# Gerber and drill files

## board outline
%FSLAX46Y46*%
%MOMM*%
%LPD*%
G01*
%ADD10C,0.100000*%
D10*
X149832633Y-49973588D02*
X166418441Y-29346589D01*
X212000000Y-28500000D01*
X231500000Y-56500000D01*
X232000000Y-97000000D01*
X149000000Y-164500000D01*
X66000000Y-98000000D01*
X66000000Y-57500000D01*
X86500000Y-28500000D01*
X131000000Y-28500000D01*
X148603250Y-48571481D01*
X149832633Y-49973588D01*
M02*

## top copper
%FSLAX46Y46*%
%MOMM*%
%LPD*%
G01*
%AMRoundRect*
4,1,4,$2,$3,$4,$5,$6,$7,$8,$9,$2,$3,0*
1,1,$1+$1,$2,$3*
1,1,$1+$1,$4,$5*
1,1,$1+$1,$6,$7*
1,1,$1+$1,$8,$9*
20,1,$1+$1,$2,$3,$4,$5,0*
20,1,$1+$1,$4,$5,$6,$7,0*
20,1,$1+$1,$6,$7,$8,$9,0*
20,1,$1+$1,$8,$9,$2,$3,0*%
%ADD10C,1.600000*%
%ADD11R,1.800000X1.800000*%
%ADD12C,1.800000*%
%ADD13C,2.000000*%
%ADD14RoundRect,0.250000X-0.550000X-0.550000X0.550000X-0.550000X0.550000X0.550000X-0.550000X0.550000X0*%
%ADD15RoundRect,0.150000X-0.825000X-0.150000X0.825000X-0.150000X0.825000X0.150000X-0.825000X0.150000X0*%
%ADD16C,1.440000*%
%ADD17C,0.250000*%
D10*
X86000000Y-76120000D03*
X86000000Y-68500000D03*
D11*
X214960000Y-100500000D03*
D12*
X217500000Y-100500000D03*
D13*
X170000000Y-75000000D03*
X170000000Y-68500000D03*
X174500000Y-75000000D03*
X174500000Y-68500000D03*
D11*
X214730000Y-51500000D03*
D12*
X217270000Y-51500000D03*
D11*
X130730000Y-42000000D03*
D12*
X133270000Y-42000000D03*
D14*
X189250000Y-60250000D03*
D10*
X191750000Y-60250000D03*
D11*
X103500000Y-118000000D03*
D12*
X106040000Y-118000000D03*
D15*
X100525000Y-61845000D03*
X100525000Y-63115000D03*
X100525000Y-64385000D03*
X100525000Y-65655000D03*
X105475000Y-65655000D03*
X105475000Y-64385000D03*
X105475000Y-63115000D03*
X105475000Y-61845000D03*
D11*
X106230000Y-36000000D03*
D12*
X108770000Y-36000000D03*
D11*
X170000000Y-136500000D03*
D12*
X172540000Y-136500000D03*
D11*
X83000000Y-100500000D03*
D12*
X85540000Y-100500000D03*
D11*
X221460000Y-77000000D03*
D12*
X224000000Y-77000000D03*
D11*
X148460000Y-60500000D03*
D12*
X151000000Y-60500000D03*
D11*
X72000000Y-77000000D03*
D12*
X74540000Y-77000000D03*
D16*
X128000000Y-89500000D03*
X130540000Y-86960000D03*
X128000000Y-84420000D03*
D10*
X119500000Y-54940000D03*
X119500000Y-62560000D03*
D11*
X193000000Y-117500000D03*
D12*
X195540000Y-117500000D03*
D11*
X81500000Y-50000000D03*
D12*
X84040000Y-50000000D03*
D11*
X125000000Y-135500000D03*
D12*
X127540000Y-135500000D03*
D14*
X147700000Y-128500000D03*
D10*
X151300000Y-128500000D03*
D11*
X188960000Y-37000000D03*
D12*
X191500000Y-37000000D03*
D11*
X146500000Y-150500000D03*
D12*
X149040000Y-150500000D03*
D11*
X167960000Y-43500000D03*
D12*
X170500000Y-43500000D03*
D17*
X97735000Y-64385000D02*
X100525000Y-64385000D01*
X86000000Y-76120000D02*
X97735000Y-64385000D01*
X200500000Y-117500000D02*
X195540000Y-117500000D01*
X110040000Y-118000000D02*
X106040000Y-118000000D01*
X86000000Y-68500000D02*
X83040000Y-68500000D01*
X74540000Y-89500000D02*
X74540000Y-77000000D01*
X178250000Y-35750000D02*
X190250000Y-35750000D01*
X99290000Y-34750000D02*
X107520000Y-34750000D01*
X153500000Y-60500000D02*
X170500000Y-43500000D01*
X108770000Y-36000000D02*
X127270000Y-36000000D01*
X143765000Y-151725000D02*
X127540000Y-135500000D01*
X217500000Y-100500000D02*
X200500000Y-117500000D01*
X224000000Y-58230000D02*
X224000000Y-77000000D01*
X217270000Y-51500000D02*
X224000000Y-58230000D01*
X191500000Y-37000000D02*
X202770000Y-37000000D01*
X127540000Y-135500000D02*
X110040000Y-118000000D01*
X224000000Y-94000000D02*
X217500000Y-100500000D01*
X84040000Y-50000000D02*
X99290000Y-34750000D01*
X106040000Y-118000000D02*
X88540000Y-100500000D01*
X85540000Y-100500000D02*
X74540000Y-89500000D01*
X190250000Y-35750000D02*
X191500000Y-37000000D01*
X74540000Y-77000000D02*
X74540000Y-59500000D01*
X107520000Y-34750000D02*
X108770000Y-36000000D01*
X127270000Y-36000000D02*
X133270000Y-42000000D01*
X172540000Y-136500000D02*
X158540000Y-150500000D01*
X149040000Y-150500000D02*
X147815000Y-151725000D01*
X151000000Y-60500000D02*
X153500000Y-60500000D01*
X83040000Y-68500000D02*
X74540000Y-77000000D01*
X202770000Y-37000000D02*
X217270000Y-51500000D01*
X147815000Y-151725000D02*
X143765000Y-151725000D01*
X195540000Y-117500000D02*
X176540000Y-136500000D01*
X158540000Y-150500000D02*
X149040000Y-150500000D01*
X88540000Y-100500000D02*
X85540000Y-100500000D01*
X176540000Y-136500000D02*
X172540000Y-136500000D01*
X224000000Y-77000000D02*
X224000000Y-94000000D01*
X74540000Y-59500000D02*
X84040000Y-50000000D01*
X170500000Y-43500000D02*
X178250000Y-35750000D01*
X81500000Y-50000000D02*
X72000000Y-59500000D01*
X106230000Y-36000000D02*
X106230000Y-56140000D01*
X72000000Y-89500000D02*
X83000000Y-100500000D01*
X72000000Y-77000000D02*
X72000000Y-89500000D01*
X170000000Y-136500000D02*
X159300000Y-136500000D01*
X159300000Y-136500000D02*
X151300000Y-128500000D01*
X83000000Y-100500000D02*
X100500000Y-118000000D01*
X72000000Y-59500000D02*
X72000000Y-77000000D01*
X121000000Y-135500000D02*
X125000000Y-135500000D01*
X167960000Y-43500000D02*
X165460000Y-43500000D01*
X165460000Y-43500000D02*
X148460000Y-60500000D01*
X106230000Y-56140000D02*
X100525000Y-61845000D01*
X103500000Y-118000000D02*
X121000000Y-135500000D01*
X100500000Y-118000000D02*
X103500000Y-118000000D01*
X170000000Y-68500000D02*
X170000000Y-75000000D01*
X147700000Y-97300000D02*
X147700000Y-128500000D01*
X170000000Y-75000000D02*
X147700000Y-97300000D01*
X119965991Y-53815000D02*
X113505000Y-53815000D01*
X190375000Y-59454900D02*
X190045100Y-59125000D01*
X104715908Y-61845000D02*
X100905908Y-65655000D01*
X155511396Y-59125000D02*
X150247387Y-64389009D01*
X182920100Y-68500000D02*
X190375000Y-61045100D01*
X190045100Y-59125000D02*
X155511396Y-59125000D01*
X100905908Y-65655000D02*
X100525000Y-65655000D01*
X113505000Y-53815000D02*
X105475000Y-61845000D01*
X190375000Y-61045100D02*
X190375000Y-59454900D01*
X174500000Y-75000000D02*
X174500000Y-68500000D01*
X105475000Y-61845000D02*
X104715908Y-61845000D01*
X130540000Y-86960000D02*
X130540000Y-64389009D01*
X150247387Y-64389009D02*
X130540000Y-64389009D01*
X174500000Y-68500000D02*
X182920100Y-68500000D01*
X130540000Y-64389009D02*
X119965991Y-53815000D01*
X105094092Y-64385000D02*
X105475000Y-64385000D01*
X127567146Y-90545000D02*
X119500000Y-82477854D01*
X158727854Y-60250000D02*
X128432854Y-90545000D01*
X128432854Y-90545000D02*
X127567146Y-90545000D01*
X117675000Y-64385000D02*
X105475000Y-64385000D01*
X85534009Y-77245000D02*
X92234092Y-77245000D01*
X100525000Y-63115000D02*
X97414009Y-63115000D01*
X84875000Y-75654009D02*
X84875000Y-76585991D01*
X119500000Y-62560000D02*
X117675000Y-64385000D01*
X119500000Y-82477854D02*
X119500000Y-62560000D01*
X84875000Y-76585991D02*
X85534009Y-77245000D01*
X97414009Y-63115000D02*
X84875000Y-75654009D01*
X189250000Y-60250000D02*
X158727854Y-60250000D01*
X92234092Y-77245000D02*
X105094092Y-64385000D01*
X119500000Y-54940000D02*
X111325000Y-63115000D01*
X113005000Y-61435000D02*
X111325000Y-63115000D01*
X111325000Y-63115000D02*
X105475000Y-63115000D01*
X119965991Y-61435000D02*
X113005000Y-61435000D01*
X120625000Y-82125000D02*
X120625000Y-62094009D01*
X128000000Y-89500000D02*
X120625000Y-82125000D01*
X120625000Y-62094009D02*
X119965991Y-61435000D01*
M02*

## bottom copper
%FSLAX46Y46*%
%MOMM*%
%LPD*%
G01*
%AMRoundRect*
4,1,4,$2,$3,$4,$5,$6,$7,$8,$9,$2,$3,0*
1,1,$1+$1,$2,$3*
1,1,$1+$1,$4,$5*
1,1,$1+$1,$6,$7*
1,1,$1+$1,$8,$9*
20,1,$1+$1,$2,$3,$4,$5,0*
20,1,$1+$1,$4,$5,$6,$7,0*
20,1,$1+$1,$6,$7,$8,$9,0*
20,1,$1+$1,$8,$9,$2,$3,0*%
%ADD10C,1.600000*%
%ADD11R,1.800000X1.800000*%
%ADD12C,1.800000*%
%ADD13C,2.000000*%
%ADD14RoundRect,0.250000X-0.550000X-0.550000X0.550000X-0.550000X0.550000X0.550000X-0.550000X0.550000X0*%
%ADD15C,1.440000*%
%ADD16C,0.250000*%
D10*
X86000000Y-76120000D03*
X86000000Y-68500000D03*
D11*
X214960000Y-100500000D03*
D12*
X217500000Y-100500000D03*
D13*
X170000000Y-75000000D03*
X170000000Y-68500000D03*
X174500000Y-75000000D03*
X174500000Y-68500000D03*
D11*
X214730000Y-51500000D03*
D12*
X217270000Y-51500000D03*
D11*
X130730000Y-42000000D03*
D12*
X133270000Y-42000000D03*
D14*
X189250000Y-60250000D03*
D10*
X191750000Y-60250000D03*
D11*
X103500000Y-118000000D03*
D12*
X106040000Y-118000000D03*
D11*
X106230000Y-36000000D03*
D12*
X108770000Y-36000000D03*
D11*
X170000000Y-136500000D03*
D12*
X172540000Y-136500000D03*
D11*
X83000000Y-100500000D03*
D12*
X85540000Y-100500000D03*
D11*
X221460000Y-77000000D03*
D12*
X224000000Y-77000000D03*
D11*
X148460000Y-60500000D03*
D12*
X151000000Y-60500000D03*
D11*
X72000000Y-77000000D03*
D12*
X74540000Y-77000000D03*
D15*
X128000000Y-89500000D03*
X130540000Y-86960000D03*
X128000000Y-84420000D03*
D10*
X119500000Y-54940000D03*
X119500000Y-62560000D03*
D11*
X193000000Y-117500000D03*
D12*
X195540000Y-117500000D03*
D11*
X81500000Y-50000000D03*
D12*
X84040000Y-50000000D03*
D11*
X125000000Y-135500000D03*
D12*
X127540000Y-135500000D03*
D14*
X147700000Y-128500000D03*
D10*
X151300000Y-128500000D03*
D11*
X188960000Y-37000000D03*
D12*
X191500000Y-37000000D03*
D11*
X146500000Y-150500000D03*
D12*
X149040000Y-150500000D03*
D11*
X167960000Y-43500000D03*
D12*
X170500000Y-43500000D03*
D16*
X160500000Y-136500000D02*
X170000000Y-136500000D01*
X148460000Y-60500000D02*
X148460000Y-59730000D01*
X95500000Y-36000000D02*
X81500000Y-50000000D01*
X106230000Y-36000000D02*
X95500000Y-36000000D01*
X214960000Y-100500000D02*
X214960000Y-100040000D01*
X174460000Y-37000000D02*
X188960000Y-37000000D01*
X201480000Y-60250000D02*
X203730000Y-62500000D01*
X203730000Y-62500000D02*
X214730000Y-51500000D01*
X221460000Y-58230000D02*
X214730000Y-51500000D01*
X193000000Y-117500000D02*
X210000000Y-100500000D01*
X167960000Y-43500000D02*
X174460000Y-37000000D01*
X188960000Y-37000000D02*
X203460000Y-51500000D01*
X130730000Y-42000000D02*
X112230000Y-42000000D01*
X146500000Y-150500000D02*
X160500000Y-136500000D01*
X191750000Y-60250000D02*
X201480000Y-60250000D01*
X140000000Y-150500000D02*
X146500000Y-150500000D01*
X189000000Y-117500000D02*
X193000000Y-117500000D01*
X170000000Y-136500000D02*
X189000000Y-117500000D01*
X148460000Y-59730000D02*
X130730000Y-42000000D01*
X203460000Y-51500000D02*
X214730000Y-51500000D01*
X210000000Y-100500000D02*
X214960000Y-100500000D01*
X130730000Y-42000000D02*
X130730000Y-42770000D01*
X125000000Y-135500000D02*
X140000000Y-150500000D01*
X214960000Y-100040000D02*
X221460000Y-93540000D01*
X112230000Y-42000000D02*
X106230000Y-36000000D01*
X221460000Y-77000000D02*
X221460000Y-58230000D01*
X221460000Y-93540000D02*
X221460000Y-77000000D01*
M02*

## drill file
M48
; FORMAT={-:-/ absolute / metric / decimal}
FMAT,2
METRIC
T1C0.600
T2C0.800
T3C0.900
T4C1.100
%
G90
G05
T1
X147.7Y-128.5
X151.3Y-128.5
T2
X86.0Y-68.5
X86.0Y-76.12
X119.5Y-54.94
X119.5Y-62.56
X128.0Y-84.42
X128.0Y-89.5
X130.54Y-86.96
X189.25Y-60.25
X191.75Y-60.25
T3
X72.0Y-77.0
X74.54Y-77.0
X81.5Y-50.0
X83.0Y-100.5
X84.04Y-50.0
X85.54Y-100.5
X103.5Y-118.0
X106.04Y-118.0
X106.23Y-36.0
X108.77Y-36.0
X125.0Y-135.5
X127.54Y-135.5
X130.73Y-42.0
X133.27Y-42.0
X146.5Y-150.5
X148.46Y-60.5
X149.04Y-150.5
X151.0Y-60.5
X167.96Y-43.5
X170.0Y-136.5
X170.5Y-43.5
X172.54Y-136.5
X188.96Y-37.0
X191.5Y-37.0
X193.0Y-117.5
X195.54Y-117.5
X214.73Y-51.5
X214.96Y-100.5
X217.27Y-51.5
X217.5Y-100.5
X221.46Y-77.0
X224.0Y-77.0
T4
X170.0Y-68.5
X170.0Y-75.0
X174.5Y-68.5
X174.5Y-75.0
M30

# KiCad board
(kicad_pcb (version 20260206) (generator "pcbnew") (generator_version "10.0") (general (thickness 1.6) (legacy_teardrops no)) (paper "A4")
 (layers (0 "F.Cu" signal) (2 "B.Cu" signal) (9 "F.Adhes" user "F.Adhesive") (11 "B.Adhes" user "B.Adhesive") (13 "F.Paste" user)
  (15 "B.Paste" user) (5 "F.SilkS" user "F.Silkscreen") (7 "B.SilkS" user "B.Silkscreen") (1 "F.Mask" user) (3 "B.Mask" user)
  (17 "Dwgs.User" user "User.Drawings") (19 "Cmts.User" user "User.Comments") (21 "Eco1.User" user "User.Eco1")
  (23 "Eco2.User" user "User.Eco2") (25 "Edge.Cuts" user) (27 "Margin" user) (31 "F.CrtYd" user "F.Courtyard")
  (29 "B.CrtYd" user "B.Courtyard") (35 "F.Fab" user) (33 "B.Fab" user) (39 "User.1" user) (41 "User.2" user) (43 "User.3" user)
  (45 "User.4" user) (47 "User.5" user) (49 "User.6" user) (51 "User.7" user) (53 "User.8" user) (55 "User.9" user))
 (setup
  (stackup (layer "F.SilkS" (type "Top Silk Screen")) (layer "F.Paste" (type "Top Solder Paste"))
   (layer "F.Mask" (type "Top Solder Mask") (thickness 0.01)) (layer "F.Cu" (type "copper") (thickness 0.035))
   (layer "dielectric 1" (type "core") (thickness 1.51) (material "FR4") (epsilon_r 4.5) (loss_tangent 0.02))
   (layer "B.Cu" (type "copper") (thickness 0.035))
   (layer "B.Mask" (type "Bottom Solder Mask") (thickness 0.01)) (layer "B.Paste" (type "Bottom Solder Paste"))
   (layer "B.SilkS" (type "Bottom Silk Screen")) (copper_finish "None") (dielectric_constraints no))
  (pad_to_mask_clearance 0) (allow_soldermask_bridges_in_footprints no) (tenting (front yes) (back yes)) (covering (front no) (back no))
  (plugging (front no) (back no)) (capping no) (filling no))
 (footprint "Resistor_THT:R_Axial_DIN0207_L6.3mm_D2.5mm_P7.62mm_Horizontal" (layer "F.Cu") (at 86 76.12 90)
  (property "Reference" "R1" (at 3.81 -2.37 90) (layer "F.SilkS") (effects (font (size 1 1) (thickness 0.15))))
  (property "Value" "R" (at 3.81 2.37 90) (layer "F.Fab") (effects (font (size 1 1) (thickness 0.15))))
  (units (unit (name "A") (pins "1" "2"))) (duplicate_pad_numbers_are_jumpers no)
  (pad "1" thru_hole circle (at 0 0 90) (size 1.6 1.6) (drill 0.8) (layers "*.Cu" "*.Mask") (remove_unused_layers no) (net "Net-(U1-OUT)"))
  (pad "2" thru_hole circle (at 7.62 0 90) (size 1.6 1.6) (drill 0.8) (layers "*.Cu" "*.Mask") (remove_unused_layers no) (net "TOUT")))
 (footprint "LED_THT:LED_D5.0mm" (layer "F.Cu") (at 214.96 100.5)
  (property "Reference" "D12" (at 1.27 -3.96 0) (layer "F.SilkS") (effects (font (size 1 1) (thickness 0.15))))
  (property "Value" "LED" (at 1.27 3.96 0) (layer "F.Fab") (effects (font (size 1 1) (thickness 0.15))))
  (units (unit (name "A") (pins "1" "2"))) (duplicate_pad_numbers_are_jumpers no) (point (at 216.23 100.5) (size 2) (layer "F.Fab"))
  (pad "1" thru_hole rect (at 0 0) (size 1.8 1.8) (drill 0.9) (layers "*.Cu" "*.Mask") (remove_unused_layers no) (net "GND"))
  (pad "2" thru_hole circle (at 2.54 0) (size 1.8 1.8) (drill 0.9) (layers "*.Cu" "*.Mask") (remove_unused_layers no) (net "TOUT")))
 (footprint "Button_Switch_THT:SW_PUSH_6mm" (layer "F.Cu") (at 170 75 90)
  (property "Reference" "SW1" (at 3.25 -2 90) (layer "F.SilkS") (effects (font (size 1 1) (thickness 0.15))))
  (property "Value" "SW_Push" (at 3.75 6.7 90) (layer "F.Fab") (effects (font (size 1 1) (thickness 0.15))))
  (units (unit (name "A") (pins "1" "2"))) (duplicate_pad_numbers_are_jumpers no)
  (pad "1" thru_hole circle (at 0 0 180) (size 2 2) (drill 1.1) (layers "*.Cu" "*.Mask") (remove_unused_layers no) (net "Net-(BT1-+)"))
  (pad "1" thru_hole circle (at 6.5 0 180) (size 2 2) (drill 1.1) (layers "*.Cu" "*.Mask") (remove_unused_layers no) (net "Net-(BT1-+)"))
  (pad "2" thru_hole circle (at 0 4.5 180) (size 2 2) (drill 1.1) (layers "*.Cu" "*.Mask") (remove_unused_layers no) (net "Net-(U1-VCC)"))
  (pad "2" thru_hole circle (at 6.5 4.5 180) (size 2 2) (drill 1.1) (layers "*.Cu" "*.Mask") (remove_unused_layers no) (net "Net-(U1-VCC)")))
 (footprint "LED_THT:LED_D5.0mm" (layer "F.Cu") (at 214.73 51.5)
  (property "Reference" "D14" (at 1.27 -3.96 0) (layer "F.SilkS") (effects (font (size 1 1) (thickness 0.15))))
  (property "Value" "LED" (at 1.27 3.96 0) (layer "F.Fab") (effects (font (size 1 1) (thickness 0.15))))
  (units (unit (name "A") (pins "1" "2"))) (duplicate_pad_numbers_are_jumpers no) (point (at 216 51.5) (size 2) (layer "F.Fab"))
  (pad "1" thru_hole rect (at 0 0) (size 1.8 1.8) (drill 0.9) (layers "*.Cu" "*.Mask") (remove_unused_layers no) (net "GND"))
  (pad "2" thru_hole circle (at 2.54 0) (size 1.8 1.8) (drill 0.9) (layers "*.Cu" "*.Mask") (remove_unused_layers no) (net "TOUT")))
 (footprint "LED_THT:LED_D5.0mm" (layer "F.Cu") (at 130.73 42)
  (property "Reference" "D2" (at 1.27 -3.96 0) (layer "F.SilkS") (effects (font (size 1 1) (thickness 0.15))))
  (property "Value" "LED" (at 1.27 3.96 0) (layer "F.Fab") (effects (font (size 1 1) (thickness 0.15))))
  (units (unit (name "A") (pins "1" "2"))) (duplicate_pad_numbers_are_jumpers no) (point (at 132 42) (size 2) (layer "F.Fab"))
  (pad "1" thru_hole rect (at 0 0) (size 1.8 1.8) (drill 0.9) (layers "*.Cu" "*.Mask") (remove_unused_layers no) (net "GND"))
  (pad "2" thru_hole circle (at 2.54 0) (size 1.8 1.8) (drill 0.9) (layers "*.Cu" "*.Mask") (remove_unused_layers no) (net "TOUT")))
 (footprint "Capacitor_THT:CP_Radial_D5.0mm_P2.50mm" (layer "F.Cu") (at 189.25 60.25)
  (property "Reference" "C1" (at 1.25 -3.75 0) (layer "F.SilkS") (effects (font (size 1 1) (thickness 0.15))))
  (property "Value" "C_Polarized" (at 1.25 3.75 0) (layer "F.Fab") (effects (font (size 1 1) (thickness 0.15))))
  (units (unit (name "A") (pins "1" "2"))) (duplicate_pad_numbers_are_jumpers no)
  (pad "1" thru_hole roundrect (at 0 0) (size 1.6 1.6) (drill 0.8) (layers "*.Cu" "*.Mask") (remove_unused_layers no)
   (roundrect_rratio 0.15625) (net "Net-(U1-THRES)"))
  (pad "2" thru_hole circle (at 2.5 0) (size 1.6 1.6) (drill 0.8) (layers "*.Cu" "*.Mask") (remove_unused_layers no) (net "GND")))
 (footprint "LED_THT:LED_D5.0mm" (layer "F.Cu") (at 103.5 118)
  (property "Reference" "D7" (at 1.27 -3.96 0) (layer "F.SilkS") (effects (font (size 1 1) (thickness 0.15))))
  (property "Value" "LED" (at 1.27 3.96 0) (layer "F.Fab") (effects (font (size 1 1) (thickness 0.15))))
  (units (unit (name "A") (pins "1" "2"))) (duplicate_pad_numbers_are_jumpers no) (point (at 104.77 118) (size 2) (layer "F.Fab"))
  (pad "1" thru_hole rect (at 0 0) (size 1.8 1.8) (drill 0.9) (layers "*.Cu" "*.Mask") (remove_unused_layers no) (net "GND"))
  (pad "2" thru_hole circle (at 2.54 0) (size 1.8 1.8) (drill 0.9) (layers "*.Cu" "*.Mask") (remove_unused_layers no) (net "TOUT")))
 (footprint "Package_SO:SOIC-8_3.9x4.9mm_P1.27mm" (layer "F.Cu") (at 103 63.75)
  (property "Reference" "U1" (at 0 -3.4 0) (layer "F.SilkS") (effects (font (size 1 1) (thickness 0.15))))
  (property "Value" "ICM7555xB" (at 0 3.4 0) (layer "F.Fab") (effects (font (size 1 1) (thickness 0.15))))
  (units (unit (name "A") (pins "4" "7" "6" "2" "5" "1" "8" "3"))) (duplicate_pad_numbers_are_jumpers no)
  (pad "1" smd roundrect (at -2.475 -1.905) (size 1.95 0.6) (layers "F.Cu" "F.Mask" "F.Paste") (roundrect_rratio 0.25) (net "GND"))
  (pad "2" smd roundrect (at -2.475 -0.635) (size 1.95 0.6) (layers "F.Cu" "F.Mask" "F.Paste") (roundrect_rratio 0.25)
   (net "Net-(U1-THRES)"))
  (pad "3" smd roundrect (at -2.475 0.635) (size 1.95 0.6) (layers "F.Cu" "F.Mask" "F.Paste") (roundrect_rratio 0.25) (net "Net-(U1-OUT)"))
  (pad "4" smd roundrect (at -2.475 1.905) (size 1.95 0.6) (layers "F.Cu" "F.Mask" "F.Paste") (roundrect_rratio 0.25) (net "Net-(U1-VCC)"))
  (pad "5" smd roundrect (at 2.475 1.905) (size 1.95 0.6) (layers "F.Cu" "F.Mask" "F.Paste") (roundrect_rratio 0.25)
   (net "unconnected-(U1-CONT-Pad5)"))
  (pad "6" smd roundrect (at 2.475 0.635) (size 1.95 0.6) (layers "F.Cu" "F.Mask" "F.Paste") (roundrect_rratio 0.25) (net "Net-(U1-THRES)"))
  (pad "7" smd roundrect (at 2.475 -0.635) (size 1.95 0.6) (layers "F.Cu" "F.Mask" "F.Paste") (roundrect_rratio 0.25) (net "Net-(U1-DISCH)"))
  (pad "8" smd roundrect (at 2.475 -1.905) (size 1.95 0.6) (layers "F.Cu" "F.Mask" "F.Paste") (roundrect_rratio 0.25) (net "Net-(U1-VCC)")))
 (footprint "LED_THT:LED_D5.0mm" (layer "F.Cu") (at 106.23 36)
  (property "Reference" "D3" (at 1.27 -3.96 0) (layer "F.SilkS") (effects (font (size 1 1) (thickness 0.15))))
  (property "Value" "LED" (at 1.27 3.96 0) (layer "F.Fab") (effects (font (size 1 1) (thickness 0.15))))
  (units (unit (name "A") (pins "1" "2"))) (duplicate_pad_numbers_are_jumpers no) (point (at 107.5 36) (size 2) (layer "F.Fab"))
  (pad "1" thru_hole rect (at 0 0) (size 1.8 1.8) (drill 0.9) (layers "*.Cu" "*.Mask") (remove_unused_layers no) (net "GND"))
  (pad "2" thru_hole circle (at 2.54 0) (size 1.8 1.8) (drill 0.9) (layers "*.Cu" "*.Mask") (remove_unused_layers no) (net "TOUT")))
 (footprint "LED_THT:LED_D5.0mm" (layer "F.Cu") (at 170 136.5)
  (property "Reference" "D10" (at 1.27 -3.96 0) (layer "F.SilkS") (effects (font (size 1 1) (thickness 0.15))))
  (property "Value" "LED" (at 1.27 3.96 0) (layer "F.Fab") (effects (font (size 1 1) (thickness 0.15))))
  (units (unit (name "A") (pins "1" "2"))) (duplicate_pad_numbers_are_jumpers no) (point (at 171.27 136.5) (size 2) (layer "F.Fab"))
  (pad "1" thru_hole rect (at 0 0) (size 1.8 1.8) (drill 0.9) (layers "*.Cu" "*.Mask") (remove_unused_layers no) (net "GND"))
  (pad "2" thru_hole circle (at 2.54 0) (size 1.8 1.8) (drill 0.9) (layers "*.Cu" "*.Mask") (remove_unused_layers no) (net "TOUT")))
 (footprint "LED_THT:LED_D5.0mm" (layer "F.Cu") (at 83 100.5)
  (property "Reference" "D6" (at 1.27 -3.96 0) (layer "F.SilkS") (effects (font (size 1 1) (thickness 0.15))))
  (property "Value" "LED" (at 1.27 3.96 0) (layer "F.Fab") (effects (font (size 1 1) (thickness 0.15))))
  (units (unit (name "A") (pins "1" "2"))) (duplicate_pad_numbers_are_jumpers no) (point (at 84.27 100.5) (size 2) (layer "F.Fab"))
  (pad "1" thru_hole rect (at 0 0) (size 1.8 1.8) (drill 0.9) (layers "*.Cu" "*.Mask") (remove_unused_layers no) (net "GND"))
  (pad "2" thru_hole circle (at 2.54 0) (size 1.8 1.8) (drill 0.9) (layers "*.Cu" "*.Mask") (remove_unused_layers no) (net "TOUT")))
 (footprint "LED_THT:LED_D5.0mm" (layer "F.Cu") (at 221.46 77)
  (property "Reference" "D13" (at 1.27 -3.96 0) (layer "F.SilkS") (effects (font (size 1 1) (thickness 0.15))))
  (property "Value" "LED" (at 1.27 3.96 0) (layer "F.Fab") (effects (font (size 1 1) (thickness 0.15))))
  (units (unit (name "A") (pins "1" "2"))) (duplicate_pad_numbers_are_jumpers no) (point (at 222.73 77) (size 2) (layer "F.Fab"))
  (pad "1" thru_hole rect (at 0 0) (size 1.8 1.8) (drill 0.9) (layers "*.Cu" "*.Mask") (remove_unused_layers no) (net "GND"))
  (pad "2" thru_hole circle (at 2.54 0) (size 1.8 1.8) (drill 0.9) (layers "*.Cu" "*.Mask") (remove_unused_layers no) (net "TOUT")))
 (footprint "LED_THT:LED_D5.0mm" (layer "F.Cu") (at 148.46 60.5)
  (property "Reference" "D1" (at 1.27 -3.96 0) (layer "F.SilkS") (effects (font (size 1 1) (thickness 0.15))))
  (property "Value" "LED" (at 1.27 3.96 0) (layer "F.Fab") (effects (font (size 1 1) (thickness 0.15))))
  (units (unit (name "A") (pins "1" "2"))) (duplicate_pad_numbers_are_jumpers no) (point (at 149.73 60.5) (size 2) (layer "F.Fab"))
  (pad "1" thru_hole rect (at 0 0) (size 1.8 1.8) (drill 0.9) (layers "*.Cu" "*.Mask") (remove_unused_layers no) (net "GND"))
  (pad "2" thru_hole circle (at 2.54 0) (size 1.8 1.8) (drill 0.9) (layers "*.Cu" "*.Mask") (remove_unused_layers no) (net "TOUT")))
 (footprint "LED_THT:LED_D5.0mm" (layer "F.Cu") (at 72 77)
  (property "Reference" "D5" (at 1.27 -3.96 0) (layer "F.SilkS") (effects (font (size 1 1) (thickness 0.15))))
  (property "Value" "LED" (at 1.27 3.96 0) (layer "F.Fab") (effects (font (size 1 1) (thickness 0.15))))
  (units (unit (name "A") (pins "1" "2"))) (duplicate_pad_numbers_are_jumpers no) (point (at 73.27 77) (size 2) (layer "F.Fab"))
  (pad "1" thru_hole rect (at 0 0) (size 1.8 1.8) (drill 0.9) (layers "*.Cu" "*.Mask") (remove_unused_layers no) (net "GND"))
  (pad "2" thru_hole circle (at 2.54 0) (size 1.8 1.8) (drill 0.9) (layers "*.Cu" "*.Mask") (remove_unused_layers no) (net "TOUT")))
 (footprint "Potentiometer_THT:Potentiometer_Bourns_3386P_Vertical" (layer "F.Cu") (at 128 89.5)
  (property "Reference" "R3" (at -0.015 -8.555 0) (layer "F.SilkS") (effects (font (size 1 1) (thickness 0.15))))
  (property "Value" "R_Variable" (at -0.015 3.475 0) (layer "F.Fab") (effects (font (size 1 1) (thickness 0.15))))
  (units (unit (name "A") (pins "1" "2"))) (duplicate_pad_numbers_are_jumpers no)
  (pad "1" thru_hole circle (at 0 0) (size 1.44 1.44) (drill 0.8) (layers "*.Cu" "*.Mask") (remove_unused_layers no) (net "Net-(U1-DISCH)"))
  (pad "2" thru_hole circle (at 2.54 -2.54) (size 1.44 1.44) (drill 0.8) (layers "*.Cu" "*.Mask") (remove_unused_layers no)
   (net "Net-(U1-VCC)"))
  (pad "3" thru_hole circle (at 0 -5.08) (size 1.44 1.44) (drill 0.8) (layers "*.Cu" "*.Mask") (remove_unused_layers no)))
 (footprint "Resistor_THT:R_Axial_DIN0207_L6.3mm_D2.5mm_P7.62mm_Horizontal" (layer "F.Cu") (at 119.5 54.94 -90)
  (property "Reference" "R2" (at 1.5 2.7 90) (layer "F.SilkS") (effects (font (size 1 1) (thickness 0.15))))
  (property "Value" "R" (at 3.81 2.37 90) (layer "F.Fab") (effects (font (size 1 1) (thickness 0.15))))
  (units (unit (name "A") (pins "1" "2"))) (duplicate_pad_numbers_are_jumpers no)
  (pad "1" thru_hole circle (at 0 0 270) (size 1.6 1.6) (drill 0.8) (layers "*.Cu" "*.Mask") (remove_unused_layers no)
   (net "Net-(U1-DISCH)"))
  (pad "2" thru_hole circle (at 7.62 0 270) (size 1.6 1.6) (drill 0.8) (layers "*.Cu" "*.Mask") (remove_unused_layers no)
   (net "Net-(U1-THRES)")))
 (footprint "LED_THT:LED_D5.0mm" (layer "F.Cu") (at 193 117.5)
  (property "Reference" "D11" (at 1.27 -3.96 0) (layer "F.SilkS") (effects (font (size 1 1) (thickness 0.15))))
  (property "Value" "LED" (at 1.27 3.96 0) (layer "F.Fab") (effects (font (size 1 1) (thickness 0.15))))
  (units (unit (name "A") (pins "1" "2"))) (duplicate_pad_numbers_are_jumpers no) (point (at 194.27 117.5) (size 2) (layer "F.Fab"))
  (pad "1" thru_hole rect (at 0 0) (size 1.8 1.8) (drill 0.9) (layers "*.Cu" "*.Mask") (remove_unused_layers no) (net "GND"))
  (pad "2" thru_hole circle (at 2.54 0) (size 1.8 1.8) (drill 0.9) (layers "*.Cu" "*.Mask") (remove_unused_layers no) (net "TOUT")))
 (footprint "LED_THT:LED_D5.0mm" (layer "F.Cu") (at 81.5 50)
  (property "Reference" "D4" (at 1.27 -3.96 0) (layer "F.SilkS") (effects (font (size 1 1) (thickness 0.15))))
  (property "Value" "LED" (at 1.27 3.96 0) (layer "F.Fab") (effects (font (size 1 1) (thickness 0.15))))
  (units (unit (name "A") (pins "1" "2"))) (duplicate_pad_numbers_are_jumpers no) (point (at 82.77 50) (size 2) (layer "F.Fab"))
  (pad "1" thru_hole rect (at 0 0) (size 1.8 1.8) (drill 0.9) (layers "*.Cu" "*.Mask") (remove_unused_layers no) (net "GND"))
  (pad "2" thru_hole circle (at 2.54 0) (size 1.8 1.8) (drill 0.9) (layers "*.Cu" "*.Mask") (remove_unused_layers no) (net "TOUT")))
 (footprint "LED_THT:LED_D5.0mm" (layer "F.Cu") (at 125 135.5)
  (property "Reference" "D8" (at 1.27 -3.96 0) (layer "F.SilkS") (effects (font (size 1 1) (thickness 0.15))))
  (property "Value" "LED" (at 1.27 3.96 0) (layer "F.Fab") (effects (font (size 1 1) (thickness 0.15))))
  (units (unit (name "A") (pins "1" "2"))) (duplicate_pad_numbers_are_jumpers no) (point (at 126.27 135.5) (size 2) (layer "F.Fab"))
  (pad "1" thru_hole rect (at 0 0) (size 1.8 1.8) (drill 0.9) (layers "*.Cu" "*.Mask") (remove_unused_layers no) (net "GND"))
  (pad "2" thru_hole circle (at 2.54 0) (size 1.8 1.8) (drill 0.9) (layers "*.Cu" "*.Mask") (remove_unused_layers no) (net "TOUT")))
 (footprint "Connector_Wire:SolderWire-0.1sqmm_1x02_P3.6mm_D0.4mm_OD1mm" (layer "F.Cu") (at 147.7 128.5)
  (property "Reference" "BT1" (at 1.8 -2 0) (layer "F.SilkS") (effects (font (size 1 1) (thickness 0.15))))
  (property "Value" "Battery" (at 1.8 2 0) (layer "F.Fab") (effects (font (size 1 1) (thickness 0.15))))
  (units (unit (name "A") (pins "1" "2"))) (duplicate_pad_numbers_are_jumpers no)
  (pad "1" thru_hole roundrect (at 0 0) (size 1.6 1.6) (drill 0.6) (layers "*.Cu" "*.Mask") (remove_unused_layers no)
   (roundrect_rratio 0.15625) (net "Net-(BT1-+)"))
  (pad "2" thru_hole circle (at 3.6 0) (size 1.6 1.6) (drill 0.6) (layers "*.Cu" "*.Mask") (remove_unused_layers no) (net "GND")))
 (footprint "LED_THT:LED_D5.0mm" (layer "F.Cu") (at 188.96 37)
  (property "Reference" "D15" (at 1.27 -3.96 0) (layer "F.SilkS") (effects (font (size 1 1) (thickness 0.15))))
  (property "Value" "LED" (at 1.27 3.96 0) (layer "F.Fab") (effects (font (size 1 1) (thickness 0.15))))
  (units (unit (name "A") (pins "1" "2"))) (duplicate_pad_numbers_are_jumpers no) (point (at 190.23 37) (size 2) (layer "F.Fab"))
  (pad "1" thru_hole rect (at 0 0) (size 1.8 1.8) (drill 0.9) (layers "*.Cu" "*.Mask") (remove_unused_layers no) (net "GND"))
  (pad "2" thru_hole circle (at 2.54 0) (size 1.8 1.8) (drill 0.9) (layers "*.Cu" "*.Mask") (remove_unused_layers no) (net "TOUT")))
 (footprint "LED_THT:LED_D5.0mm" (layer "F.Cu") (at 146.5 150.5)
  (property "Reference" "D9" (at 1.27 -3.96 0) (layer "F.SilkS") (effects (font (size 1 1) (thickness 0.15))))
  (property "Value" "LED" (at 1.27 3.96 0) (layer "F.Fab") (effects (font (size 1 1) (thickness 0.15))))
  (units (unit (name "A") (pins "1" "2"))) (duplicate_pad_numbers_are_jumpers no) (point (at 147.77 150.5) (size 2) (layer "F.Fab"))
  (pad "1" thru_hole rect (at 0 0) (size 1.8 1.8) (drill 0.9) (layers "*.Cu" "*.Mask") (remove_unused_layers no) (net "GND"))
  (pad "2" thru_hole circle (at 2.54 0) (size 1.8 1.8) (drill 0.9) (layers "*.Cu" "*.Mask") (remove_unused_layers no) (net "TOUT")))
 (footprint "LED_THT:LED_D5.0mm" (layer "F.Cu") (at 167.96 43.5)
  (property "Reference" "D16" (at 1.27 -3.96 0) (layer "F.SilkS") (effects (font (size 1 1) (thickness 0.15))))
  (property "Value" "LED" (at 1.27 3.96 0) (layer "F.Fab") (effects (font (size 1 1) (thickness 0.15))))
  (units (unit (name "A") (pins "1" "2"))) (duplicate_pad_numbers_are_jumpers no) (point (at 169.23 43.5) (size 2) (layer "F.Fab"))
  (pad "1" thru_hole rect (at 0 0) (size 1.8 1.8) (drill 0.9) (layers "*.Cu" "*.Mask") (remove_unused_layers no) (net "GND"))
  (pad "2" thru_hole circle (at 2.54 0) (size 1.8 1.8) (drill 0.9) (layers "*.Cu" "*.Mask") (remove_unused_layers no) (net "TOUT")))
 (gr_poly
  (pts (xy 149.832633 49.973588) (xy 166.418441 29.346589) (xy 212 28.5) (xy 231.5 56.5) (xy 232 97) (xy 149 164.5) (xy 66 98) (xy 66 57.5)
   (xy 86.5 28.5) (xy 131 28.5) (xy 148.60325 48.571481))
  (stroke (width 0.1) (type solid)) (fill no) (layer "Edge.Cuts"))
 (segment (start 97.735 64.385) (end 100.525 64.385) (width 0.25) (layer "F.Cu") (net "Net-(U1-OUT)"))
 (segment (start 86 76.12) (end 97.735 64.385) (width 0.25) (layer "F.Cu") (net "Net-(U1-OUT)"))
 (segment (start 200.5 117.5) (end 195.54 117.5) (width 0.25) (layer "F.Cu") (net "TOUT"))
 (segment (start 110.04 118) (end 106.04 118) (width 0.25) (layer "F.Cu") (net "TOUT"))
 (segment (start 86 68.5) (end 83.04 68.5) (width 0.25) (layer "F.Cu") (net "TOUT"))
 (segment (start 74.54 89.5) (end 74.54 77) (width 0.25) (layer "F.Cu") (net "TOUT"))
 (segment (start 178.25 35.75) (end 190.25 35.75) (width 0.25) (layer "F.Cu") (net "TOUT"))
 (segment (start 99.29 34.75) (end 107.52 34.75) (width 0.25) (layer "F.Cu") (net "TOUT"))
 (segment (start 153.5 60.5) (end 170.5 43.5) (width 0.25) (layer "F.Cu") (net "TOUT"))
 (segment (start 108.77 36) (end 127.27 36) (width 0.25) (layer "F.Cu") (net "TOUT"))
 (segment (start 143.765 151.725) (end 127.54 135.5) (width 0.25) (layer "F.Cu") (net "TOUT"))
 (segment (start 217.5 100.5) (end 200.5 117.5) (width 0.25) (layer "F.Cu") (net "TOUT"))
 (segment (start 224 58.23) (end 224 77) (width 0.25) (layer "F.Cu") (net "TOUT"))
 (segment (start 217.27 51.5) (end 224 58.23) (width 0.25) (layer "F.Cu") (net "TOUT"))
 (segment (start 191.5 37) (end 202.77 37) (width 0.25) (layer "F.Cu") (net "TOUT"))
 (segment (start 127.54 135.5) (end 110.04 118) (width 0.25) (layer "F.Cu") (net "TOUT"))
 (segment (start 224 94) (end 217.5 100.5) (width 0.25) (layer "F.Cu") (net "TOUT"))
 (segment (start 84.04 50) (end 99.29 34.75) (width 0.25) (layer "F.Cu") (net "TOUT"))
 (segment (start 106.04 118) (end 88.54 100.5) (width 0.25) (layer "F.Cu") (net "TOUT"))
 (segment (start 85.54 100.5) (end 74.54 89.5) (width 0.25) (layer "F.Cu") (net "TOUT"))
 (segment (start 190.25 35.75) (end 191.5 37) (width 0.25) (layer "F.Cu") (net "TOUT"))
 (segment (start 74.54 77) (end 74.54 59.5) (width 0.25) (layer "F.Cu") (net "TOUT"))
 (segment (start 107.52 34.75) (end 108.77 36) (width 0.25) (layer "F.Cu") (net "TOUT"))
 (segment (start 127.27 36) (end 133.27 42) (width 0.25) (layer "F.Cu") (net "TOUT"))
 (segment (start 172.54 136.5) (end 158.54 150.5) (width 0.25) (layer "F.Cu") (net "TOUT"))
 (segment (start 149.04 150.5) (end 147.815 151.725) (width 0.25) (layer "F.Cu") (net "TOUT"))
 (segment (start 151 60.5) (end 153.5 60.5) (width 0.25) (layer "F.Cu") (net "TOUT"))
 (segment (start 83.04 68.5) (end 74.54 77) (width 0.25) (layer "F.Cu") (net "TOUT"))
 (segment (start 202.77 37) (end 217.27 51.5) (width 0.25) (layer "F.Cu") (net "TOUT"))
 (segment (start 147.815 151.725) (end 143.765 151.725) (width 0.25) (layer "F.Cu") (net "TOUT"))
 (segment (start 195.54 117.5) (end 176.54 136.5) (width 0.25) (layer "F.Cu") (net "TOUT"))
 (segment (start 158.54 150.5) (end 149.04 150.5) (width 0.25) (layer "F.Cu") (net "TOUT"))
 (segment (start 88.54 100.5) (end 85.54 100.5) (width 0.25) (layer "F.Cu") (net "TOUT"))
 (segment (start 176.54 136.5) (end 172.54 136.5) (width 0.25) (layer "F.Cu") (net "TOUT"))
 (segment (start 224 77) (end 224 94) (width 0.25) (layer "F.Cu") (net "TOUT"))
 (segment (start 74.54 59.5) (end 84.04 50) (width 0.25) (layer "F.Cu") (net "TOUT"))
 (segment (start 170.5 43.5) (end 178.25 35.75) (width 0.25) (layer "F.Cu") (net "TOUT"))
 (segment (start 81.5 50) (end 72 59.5) (width 0.25) (layer "F.Cu") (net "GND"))
 (segment (start 106.23 36) (end 106.23 56.14) (width 0.25) (layer "F.Cu") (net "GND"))
 (segment (start 72 89.5) (end 83 100.5) (width 0.25) (layer "F.Cu") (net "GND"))
 (segment (start 72 77) (end 72 89.5) (width 0.25) (layer "F.Cu") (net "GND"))
 (segment (start 170 136.5) (end 159.3 136.5) (width 0.25) (layer "F.Cu") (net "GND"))
 (segment (start 159.3 136.5) (end 151.3 128.5) (width 0.25) (layer "F.Cu") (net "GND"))
 (segment (start 83 100.5) (end 100.5 118) (width 0.25) (layer "F.Cu") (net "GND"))
 (segment (start 72 59.5) (end 72 77) (width 0.25) (layer "F.Cu") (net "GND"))
 (segment (start 121 135.5) (end 125 135.5) (width 0.25) (layer "F.Cu") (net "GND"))
 (segment (start 167.96 43.5) (end 165.46 43.5) (width 0.25) (layer "F.Cu") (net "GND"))
 (segment (start 165.46 43.5) (end 148.46 60.5) (width 0.25) (layer "F.Cu") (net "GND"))
 (segment (start 106.23 56.14) (end 100.525 61.845) (width 0.25) (layer "F.Cu") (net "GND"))
 (segment (start 103.5 118) (end 121 135.5) (width 0.25) (layer "F.Cu") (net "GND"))
 (segment (start 100.5 118) (end 103.5 118) (width 0.25) (layer "F.Cu") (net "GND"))
 (segment (start 160.5 136.5) (end 170 136.5) (width 0.25) (layer "B.Cu") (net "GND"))
 (segment (start 148.46 60.5) (end 148.46 59.73) (width 0.25) (layer "B.Cu") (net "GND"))
 (segment (start 95.5 36) (end 81.5 50) (width 0.25) (layer "B.Cu") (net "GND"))
 (segment (start 106.23 36) (end 95.5 36) (width 0.25) (layer "B.Cu") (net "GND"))
 (segment (start 214.96 100.5) (end 214.96 100.04) (width 0.25) (layer "B.Cu") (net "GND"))
 (segment (start 174.46 37) (end 188.96 37) (width 0.25) (layer "B.Cu") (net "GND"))
 (segment (start 201.48 60.25) (end 203.73 62.5) (width 0.25) (layer "B.Cu") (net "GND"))
 (segment (start 203.73 62.5) (end 214.73 51.5) (width 0.25) (layer "B.Cu") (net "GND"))
 (segment (start 221.46 58.23) (end 214.73 51.5) (width 0.25) (layer "B.Cu") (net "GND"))
 (segment (start 193 117.5) (end 210 100.5) (width 0.25) (layer "B.Cu") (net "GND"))
 (segment (start 167.96 43.5) (end 174.46 37) (width 0.25) (layer "B.Cu") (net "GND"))
 (segment (start 188.96 37) (end 203.46 51.5) (width 0.25) (layer "B.Cu") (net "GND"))
 (segment (start 130.73 42) (end 112.23 42) (width 0.25) (layer "B.Cu") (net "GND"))
 (segment (start 146.5 150.5) (end 160.5 136.5) (width 0.25) (layer "B.Cu") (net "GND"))
 (segment (start 191.75 60.25) (end 201.48 60.25) (width 0.25) (layer "B.Cu") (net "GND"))
 (segment (start 140 150.5) (end 146.5 150.5) (width 0.25) (layer "B.Cu") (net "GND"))
 (segment (start 189 117.5) (end 193 117.5) (width 0.25) (layer "B.Cu") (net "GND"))
 (segment (start 170 136.5) (end 189 117.5) (width 0.25) (layer "B.Cu") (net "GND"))
 (segment (start 148.46 59.73) (end 130.73 42) (width 0.25) (layer "B.Cu") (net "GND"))
 (segment (start 203.46 51.5) (end 214.73 51.5) (width 0.25) (layer "B.Cu") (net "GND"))
 (segment (start 210 100.5) (end 214.96 100.5) (width 0.25) (layer "B.Cu") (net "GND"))
 (segment (start 130.73 42) (end 130.73 42.77) (width 0.25) (layer "B.Cu") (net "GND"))
 (segment (start 125 135.5) (end 140 150.5) (width 0.25) (layer "B.Cu") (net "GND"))
 (segment (start 214.96 100.04) (end 221.46 93.54) (width 0.25) (layer "B.Cu") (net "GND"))
 (segment (start 112.23 42) (end 106.23 36) (width 0.25) (layer "B.Cu") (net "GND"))
 (segment (start 221.46 77) (end 221.46 58.23) (width 0.25) (layer "B.Cu") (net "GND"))
 (segment (start 221.46 93.54) (end 221.46 77) (width 0.25) (layer "B.Cu") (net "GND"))
 (segment (start 170 68.5) (end 170 75) (width 0.25) (layer "F.Cu") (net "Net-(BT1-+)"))
 (segment (start 147.7 97.3) (end 147.7 128.5) (width 0.25) (layer "F.Cu") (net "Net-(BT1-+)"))
 (segment (start 170 75) (end 147.7 97.3) (width 0.25) (layer "F.Cu") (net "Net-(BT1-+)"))
 (segment (start 119.965991 53.815) (end 113.505 53.815) (width 0.25) (layer "F.Cu") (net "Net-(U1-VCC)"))
 (segment (start 190.375 59.4549) (end 190.0451 59.125) (width 0.25) (layer "F.Cu") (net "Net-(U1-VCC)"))
 (segment (start 104.715908 61.845) (end 100.905908 65.655) (width 0.25) (layer "F.Cu") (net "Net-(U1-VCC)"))
 (segment (start 155.511396 59.125) (end 150.247387 64.389009) (width 0.25) (layer "F.Cu") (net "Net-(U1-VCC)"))
 (segment (start 182.9201 68.5) (end 190.375 61.0451) (width 0.25) (layer "F.Cu") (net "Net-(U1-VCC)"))
 (segment (start 190.0451 59.125) (end 155.511396 59.125) (width 0.25) (layer "F.Cu") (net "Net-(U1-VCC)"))
 (segment (start 100.905908 65.655) (end 100.525 65.655) (width 0.25) (layer "F.Cu") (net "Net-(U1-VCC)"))
 (segment (start 113.505 53.815) (end 105.475 61.845) (width 0.25) (layer "F.Cu") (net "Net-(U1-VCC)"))
 (segment (start 190.375 61.0451) (end 190.375 59.4549) (width 0.25) (layer "F.Cu") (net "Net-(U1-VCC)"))
 (segment (start 174.5 75) (end 174.5 68.5) (width 0.25) (layer "F.Cu") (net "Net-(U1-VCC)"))
 (segment (start 105.475 61.845) (end 104.715908 61.845) (width 0.25) (layer "F.Cu") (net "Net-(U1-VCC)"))
 (segment (start 130.54 86.96) (end 130.54 64.389009) (width 0.25) (layer "F.Cu") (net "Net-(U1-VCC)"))
 (segment (start 150.247387 64.389009) (end 130.54 64.389009) (width 0.25) (layer "F.Cu") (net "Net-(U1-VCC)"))
 (segment (start 174.5 68.5) (end 182.9201 68.5) (width 0.25) (layer "F.Cu") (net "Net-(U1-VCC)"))
 (segment (start 130.54 64.389009) (end 119.965991 53.815) (width 0.25) (layer "F.Cu") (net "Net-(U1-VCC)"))
 (segment (start 105.094092 64.385) (end 105.475 64.385) (width 0.25) (layer "F.Cu") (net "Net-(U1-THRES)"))
 (segment (start 127.567146 90.545) (end 119.5 82.477854) (width 0.25) (layer "F.Cu") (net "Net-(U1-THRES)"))
 (segment (start 158.727854 60.25) (end 128.432854 90.545) (width 0.25) (layer "F.Cu") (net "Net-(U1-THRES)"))
 (segment (start 128.432854 90.545) (end 127.567146 90.545) (width 0.25) (layer "F.Cu") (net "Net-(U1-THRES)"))
 (segment (start 117.675 64.385) (end 105.475 64.385) (width 0.25) (layer "F.Cu") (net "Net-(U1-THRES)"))
 (segment (start 85.534009 77.245) (end 92.234092 77.245) (width 0.25) (layer "F.Cu") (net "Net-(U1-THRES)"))
 (segment (start 100.525 63.115) (end 97.414009 63.115) (width 0.25) (layer "F.Cu") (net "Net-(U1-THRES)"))
 (segment (start 84.875 75.654009) (end 84.875 76.585991) (width 0.25) (layer "F.Cu") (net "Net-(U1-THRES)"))
 (segment (start 119.5 62.56) (end 117.675 64.385) (width 0.25) (layer "F.Cu") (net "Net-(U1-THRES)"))
 (segment (start 119.5 82.477854) (end 119.5 62.56) (width 0.25) (layer "F.Cu") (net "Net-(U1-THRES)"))
 (segment (start 84.875 76.585991) (end 85.534009 77.245) (width 0.25) (layer "F.Cu") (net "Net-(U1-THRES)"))
 (segment (start 97.414009 63.115) (end 84.875 75.654009) (width 0.25) (layer "F.Cu") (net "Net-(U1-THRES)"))
 (segment (start 189.25 60.25) (end 158.727854 60.25) (width 0.25) (layer "F.Cu") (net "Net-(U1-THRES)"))
 (segment (start 92.234092 77.245) (end 105.094092 64.385) (width 0.25) (layer "F.Cu") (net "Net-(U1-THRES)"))
 (segment (start 119.5 54.94) (end 111.325 63.115) (width 0.25) (layer "F.Cu") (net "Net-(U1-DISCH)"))
 (segment (start 113.005 61.435) (end 111.325 63.115) (width 0.25) (layer "F.Cu") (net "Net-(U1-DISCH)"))
 (segment (start 111.325 63.115) (end 105.475 63.115) (width 0.25) (layer "F.Cu") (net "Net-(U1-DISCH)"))
 (segment (start 119.965991 61.435) (end 113.005 61.435) (width 0.25) (layer "F.Cu") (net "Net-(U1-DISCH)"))
 (segment (start 120.625 82.125) (end 120.625 62.094009) (width 0.25) (layer "F.Cu") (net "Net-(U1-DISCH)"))
 (segment (start 128 89.5) (end 120.625 82.125) (width 0.25) (layer "F.Cu") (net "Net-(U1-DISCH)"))
 (segment (start 120.625 62.094009) (end 119.965991 61.435) (width 0.25) (layer "F.Cu") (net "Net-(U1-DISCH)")))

